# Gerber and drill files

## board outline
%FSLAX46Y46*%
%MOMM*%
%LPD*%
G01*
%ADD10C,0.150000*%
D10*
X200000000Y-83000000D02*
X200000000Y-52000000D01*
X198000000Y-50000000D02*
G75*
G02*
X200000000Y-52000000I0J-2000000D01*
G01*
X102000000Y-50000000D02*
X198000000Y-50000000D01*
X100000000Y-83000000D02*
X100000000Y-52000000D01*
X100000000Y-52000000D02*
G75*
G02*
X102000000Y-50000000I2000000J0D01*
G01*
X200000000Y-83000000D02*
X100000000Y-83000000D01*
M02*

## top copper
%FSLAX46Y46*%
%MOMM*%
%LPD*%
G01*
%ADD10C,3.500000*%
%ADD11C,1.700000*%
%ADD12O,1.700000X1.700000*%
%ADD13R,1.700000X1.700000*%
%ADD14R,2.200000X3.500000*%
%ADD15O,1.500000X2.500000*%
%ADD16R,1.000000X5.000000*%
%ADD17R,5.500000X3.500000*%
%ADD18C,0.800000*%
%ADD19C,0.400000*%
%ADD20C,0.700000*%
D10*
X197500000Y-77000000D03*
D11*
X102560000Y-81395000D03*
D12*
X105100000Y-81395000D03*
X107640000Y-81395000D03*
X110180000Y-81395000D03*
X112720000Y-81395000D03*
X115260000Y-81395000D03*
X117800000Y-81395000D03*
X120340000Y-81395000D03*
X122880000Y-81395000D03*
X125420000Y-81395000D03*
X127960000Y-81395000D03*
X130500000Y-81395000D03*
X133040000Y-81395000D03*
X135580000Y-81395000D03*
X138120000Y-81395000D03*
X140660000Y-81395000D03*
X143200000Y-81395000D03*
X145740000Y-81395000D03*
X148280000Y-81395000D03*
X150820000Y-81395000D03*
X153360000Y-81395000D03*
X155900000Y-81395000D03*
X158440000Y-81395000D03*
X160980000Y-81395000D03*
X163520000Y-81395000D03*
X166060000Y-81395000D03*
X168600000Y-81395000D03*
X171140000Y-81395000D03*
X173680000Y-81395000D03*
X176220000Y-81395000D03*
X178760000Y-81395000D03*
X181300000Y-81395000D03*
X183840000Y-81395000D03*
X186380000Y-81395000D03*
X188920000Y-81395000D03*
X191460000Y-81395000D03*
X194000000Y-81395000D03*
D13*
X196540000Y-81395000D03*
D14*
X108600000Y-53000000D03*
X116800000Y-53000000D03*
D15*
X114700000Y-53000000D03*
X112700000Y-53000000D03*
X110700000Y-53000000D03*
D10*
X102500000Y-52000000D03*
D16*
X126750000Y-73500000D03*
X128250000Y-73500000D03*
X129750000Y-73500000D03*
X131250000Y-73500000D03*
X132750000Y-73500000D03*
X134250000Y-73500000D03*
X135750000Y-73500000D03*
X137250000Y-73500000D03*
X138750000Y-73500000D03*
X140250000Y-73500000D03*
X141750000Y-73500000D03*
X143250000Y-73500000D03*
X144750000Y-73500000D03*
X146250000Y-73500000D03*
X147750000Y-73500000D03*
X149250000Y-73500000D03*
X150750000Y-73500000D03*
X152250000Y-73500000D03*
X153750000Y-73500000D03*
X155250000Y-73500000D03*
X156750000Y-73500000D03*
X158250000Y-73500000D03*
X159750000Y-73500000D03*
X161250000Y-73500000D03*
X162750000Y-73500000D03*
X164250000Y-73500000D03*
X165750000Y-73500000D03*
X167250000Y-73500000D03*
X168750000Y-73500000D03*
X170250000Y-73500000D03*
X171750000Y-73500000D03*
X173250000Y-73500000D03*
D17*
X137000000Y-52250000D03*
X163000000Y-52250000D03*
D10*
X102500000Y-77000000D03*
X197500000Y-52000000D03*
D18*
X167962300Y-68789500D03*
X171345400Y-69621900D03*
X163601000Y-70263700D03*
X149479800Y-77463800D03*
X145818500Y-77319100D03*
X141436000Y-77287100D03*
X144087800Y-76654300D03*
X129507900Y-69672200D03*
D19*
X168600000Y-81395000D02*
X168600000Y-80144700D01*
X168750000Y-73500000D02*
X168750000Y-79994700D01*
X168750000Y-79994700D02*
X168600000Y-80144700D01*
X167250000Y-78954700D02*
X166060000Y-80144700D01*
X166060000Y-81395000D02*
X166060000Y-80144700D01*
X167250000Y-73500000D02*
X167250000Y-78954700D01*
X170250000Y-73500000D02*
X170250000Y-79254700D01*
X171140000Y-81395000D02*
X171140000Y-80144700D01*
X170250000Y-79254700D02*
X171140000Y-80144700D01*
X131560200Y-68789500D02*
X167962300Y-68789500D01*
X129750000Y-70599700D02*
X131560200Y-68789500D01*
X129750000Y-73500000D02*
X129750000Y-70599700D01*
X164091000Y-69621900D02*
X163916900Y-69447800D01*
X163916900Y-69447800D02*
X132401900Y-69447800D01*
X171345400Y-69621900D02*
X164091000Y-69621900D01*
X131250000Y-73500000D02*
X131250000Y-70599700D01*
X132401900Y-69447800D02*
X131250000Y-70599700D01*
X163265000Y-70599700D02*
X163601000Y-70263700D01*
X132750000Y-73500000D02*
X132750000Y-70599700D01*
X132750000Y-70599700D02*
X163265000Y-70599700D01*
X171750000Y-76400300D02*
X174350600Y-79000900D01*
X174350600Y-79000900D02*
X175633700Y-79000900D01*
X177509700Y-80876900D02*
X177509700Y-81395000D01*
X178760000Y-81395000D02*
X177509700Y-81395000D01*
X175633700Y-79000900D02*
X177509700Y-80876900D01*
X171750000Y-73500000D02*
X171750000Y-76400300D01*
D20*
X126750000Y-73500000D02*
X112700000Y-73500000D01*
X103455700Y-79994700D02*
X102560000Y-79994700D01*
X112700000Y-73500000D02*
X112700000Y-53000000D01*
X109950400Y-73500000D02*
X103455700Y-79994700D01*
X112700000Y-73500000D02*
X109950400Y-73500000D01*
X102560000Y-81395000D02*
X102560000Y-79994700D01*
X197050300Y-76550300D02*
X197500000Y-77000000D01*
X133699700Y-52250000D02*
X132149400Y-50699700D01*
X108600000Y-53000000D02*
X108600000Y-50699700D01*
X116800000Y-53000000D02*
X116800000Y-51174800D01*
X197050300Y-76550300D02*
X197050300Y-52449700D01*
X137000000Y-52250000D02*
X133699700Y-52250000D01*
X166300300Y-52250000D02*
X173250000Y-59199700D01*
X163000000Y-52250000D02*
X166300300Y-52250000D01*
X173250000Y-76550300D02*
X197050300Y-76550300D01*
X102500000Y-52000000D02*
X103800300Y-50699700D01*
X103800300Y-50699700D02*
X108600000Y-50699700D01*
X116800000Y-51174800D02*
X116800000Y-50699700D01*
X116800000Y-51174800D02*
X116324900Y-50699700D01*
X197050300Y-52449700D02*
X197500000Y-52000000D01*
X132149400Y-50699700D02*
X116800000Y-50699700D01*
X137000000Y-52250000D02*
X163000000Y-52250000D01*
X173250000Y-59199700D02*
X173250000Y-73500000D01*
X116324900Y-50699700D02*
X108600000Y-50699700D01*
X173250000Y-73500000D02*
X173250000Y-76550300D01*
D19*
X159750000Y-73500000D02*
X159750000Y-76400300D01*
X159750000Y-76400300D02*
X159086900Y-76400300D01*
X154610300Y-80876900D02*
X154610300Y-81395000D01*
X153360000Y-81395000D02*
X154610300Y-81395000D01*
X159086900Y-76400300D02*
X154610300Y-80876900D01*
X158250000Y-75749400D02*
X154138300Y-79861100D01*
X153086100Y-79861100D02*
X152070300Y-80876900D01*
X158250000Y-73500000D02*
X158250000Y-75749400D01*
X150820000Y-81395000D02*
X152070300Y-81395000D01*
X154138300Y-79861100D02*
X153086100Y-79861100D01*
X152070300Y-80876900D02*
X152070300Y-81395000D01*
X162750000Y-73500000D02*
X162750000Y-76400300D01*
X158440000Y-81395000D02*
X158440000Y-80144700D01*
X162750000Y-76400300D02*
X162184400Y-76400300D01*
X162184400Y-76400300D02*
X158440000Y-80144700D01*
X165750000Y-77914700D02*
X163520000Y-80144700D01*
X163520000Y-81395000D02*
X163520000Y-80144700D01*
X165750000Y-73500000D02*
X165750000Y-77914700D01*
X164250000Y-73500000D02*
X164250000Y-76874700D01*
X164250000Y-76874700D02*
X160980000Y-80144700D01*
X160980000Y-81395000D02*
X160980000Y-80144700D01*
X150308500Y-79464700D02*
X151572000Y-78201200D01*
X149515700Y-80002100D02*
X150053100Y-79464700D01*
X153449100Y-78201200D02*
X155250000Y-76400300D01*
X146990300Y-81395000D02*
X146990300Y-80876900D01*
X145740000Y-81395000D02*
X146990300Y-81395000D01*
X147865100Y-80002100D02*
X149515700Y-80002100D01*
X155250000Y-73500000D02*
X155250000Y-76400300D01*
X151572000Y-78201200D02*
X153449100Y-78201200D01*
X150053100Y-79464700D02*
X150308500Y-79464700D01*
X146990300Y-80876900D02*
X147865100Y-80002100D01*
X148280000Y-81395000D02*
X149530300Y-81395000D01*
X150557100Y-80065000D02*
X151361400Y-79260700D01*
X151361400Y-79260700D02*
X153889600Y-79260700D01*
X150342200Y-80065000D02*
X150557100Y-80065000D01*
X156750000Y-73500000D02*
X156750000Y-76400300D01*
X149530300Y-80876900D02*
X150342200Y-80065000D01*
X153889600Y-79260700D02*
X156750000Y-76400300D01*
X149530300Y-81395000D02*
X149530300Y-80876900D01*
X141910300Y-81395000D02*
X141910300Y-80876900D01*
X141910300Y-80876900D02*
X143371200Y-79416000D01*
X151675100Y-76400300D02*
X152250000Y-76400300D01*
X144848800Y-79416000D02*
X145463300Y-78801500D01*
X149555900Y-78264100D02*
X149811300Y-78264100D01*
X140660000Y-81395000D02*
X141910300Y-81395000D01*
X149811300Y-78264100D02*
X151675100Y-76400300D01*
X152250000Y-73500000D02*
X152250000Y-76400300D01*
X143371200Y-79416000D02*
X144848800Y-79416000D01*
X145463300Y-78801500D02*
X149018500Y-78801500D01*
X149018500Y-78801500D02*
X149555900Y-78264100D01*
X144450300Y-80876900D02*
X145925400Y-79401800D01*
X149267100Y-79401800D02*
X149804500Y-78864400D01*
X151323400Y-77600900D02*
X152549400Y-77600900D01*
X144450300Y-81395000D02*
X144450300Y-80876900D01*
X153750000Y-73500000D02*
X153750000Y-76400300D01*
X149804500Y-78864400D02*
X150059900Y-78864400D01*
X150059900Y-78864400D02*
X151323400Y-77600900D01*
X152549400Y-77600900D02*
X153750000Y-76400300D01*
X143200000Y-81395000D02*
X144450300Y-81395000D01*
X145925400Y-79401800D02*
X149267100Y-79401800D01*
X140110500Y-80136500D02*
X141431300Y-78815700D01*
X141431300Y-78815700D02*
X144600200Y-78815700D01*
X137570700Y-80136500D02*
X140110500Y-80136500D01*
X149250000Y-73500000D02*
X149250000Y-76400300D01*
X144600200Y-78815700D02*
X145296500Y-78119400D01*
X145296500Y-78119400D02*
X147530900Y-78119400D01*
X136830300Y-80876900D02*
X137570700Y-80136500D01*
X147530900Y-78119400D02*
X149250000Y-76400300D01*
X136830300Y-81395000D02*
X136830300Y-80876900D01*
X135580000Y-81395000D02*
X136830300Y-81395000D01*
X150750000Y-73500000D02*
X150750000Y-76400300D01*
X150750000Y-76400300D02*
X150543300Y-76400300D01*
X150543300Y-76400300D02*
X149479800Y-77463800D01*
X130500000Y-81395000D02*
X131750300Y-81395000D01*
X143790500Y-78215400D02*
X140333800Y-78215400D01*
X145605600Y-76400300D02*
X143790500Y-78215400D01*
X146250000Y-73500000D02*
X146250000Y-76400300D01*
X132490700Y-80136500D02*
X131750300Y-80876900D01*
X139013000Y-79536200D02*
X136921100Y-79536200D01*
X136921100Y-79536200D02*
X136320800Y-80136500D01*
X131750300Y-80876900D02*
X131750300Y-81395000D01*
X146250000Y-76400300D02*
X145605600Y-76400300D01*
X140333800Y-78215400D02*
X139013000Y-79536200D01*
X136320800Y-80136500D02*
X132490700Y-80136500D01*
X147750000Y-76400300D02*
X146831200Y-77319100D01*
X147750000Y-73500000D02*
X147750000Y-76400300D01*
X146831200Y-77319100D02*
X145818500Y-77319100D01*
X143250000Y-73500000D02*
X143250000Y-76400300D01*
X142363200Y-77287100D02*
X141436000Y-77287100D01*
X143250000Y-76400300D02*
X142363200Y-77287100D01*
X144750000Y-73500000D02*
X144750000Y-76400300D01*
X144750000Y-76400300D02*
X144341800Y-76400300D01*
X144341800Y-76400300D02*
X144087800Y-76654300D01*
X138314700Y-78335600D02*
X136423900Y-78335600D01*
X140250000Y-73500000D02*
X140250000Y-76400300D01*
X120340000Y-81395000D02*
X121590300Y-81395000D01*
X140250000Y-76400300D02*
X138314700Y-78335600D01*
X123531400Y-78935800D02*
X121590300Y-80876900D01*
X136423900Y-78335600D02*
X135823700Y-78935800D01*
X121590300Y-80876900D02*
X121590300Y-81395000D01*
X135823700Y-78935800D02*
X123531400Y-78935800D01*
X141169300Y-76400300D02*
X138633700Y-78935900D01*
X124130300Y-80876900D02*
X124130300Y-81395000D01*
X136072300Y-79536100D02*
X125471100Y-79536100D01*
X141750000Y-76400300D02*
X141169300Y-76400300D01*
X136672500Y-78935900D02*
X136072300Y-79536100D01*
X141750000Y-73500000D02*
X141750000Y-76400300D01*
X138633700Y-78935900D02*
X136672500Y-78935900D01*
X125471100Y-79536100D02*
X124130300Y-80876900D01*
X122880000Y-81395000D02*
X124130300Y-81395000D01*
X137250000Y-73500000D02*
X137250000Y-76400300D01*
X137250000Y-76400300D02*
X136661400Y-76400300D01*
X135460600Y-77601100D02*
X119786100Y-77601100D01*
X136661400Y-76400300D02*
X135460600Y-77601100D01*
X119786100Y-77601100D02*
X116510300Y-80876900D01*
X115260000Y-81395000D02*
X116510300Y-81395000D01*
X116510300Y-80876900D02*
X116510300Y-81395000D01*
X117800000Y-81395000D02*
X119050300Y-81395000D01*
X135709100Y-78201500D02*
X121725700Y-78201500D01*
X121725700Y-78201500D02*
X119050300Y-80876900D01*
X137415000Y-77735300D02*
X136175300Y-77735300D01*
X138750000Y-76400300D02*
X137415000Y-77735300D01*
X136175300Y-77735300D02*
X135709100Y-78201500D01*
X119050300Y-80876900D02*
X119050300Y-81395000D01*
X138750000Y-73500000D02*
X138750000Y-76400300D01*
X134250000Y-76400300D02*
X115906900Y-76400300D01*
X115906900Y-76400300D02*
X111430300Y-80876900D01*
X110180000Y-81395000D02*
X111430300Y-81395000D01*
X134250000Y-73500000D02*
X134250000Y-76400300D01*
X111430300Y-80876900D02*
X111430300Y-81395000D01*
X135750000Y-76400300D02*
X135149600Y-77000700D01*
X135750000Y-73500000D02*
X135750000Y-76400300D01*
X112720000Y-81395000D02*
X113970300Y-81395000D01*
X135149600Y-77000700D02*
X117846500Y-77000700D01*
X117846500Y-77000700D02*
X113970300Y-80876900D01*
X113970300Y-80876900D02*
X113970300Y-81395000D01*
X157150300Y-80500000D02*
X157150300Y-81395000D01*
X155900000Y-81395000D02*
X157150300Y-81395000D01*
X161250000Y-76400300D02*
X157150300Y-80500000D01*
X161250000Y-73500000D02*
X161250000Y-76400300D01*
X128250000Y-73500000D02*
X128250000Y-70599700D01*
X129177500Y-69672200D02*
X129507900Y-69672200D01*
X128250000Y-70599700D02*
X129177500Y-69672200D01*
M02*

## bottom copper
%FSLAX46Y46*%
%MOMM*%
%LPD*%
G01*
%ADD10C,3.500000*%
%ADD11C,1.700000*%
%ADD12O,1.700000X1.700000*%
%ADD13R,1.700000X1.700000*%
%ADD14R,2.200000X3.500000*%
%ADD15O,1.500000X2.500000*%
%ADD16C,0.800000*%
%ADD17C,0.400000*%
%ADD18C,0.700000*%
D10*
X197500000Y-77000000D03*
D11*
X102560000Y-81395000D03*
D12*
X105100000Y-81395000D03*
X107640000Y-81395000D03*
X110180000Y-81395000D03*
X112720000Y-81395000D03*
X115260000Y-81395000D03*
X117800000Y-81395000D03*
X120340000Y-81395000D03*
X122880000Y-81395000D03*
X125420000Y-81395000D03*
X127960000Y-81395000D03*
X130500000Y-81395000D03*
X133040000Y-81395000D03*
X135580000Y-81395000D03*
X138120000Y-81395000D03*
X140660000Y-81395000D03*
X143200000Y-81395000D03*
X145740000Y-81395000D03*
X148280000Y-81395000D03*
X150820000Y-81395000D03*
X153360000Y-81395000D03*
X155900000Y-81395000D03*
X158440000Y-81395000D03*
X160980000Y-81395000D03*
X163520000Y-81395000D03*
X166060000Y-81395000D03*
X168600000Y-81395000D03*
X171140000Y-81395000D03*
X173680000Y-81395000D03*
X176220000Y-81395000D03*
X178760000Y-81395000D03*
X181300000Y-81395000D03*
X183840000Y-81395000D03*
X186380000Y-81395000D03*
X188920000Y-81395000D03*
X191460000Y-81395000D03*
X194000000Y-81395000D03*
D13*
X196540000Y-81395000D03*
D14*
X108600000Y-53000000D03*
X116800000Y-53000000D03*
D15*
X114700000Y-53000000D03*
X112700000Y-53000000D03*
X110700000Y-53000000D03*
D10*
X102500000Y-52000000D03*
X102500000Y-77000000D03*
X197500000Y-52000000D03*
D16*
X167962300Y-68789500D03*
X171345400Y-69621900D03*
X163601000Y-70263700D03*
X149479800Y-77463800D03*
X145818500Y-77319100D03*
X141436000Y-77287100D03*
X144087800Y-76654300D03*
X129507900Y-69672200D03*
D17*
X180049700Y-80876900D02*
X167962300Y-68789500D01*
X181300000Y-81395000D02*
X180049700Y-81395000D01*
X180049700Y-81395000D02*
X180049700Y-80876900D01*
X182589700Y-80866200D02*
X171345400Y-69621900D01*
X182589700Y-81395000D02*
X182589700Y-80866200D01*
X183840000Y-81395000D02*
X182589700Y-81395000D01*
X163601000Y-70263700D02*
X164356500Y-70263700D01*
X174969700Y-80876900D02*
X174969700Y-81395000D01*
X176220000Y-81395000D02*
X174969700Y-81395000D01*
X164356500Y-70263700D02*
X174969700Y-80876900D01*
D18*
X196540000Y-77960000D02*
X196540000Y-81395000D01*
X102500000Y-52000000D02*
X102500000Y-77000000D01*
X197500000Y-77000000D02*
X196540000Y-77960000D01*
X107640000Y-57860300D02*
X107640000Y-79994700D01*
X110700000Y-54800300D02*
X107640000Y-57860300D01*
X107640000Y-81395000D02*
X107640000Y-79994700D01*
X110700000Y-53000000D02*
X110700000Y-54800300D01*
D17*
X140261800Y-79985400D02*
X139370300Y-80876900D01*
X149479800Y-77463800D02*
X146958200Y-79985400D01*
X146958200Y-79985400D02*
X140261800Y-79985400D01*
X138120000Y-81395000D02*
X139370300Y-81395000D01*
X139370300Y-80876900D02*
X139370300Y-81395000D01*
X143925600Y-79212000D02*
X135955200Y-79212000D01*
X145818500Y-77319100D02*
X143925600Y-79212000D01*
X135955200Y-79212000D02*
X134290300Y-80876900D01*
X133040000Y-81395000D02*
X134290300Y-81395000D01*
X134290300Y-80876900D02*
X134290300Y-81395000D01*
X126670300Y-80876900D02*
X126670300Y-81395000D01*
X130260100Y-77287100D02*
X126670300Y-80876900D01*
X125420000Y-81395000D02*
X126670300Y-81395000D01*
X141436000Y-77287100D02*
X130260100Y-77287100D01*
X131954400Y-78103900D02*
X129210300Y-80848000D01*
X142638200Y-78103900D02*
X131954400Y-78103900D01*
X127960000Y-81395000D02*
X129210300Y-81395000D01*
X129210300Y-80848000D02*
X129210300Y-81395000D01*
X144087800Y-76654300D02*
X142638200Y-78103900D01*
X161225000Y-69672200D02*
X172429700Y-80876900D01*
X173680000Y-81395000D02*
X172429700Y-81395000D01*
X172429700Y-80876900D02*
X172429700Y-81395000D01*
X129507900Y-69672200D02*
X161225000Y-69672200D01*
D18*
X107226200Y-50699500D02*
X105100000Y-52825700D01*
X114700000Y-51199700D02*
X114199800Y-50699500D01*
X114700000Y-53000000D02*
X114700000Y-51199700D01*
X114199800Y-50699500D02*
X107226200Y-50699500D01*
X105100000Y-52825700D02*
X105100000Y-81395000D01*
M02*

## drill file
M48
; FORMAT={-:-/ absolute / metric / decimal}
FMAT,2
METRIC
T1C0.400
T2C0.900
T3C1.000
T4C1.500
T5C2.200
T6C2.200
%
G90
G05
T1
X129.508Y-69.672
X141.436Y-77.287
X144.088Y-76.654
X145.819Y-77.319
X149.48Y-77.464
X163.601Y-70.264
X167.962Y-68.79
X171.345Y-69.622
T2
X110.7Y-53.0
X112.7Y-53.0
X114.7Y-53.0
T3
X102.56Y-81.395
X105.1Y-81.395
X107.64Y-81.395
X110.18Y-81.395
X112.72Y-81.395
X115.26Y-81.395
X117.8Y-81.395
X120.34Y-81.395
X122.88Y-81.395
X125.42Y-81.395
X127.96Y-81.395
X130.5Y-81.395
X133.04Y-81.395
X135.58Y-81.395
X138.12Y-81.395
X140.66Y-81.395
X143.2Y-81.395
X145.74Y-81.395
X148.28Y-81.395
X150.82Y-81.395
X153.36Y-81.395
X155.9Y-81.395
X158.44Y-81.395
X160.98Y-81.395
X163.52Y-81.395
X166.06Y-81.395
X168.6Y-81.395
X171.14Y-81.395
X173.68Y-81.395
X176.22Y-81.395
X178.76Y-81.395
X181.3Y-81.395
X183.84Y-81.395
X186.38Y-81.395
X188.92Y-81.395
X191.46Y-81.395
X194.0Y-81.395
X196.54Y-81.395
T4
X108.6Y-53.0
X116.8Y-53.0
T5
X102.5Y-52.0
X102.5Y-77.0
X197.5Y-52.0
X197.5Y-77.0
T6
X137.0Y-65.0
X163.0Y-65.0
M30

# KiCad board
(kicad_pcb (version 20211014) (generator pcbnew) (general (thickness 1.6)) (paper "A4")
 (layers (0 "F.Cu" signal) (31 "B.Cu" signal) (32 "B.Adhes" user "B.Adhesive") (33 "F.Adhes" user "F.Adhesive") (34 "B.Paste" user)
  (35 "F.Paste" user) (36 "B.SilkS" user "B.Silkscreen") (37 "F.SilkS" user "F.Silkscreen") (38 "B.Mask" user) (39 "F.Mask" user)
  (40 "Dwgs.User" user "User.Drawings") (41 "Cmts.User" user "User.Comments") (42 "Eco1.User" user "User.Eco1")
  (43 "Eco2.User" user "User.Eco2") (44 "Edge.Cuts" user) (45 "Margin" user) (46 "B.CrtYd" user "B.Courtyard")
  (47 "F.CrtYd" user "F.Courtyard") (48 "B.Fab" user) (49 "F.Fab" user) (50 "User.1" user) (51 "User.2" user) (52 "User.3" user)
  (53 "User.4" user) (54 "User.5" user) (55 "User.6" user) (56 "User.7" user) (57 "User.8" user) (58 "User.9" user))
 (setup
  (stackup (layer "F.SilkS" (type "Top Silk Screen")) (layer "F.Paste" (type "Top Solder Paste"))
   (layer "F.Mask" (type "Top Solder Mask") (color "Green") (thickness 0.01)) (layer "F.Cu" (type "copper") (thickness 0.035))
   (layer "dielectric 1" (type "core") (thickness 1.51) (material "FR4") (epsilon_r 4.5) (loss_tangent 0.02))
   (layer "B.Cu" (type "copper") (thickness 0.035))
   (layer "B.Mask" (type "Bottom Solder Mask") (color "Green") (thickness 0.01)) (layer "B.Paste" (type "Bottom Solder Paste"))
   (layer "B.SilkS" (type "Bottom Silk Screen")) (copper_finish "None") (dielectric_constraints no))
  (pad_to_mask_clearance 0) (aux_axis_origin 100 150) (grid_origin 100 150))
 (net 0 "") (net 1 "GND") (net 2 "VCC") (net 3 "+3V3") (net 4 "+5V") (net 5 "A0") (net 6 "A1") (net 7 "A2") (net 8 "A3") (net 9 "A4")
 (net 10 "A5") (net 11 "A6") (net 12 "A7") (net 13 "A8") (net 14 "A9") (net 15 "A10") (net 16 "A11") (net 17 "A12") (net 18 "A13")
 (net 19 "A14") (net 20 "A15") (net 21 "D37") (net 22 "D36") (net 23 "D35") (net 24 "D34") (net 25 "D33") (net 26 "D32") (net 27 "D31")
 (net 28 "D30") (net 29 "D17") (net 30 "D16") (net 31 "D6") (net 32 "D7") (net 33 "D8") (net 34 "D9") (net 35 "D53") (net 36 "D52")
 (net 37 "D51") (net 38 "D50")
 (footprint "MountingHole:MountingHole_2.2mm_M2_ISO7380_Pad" (layer "F.Cu") (at 197.5 77)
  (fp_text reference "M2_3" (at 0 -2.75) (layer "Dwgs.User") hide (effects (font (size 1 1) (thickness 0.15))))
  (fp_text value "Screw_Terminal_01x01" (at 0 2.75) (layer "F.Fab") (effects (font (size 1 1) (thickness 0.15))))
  (pad "1" thru_hole circle locked (at 0 0) (size 3.5 3.5) (drill 2.2) (layers *.Cu *.Mask) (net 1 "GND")))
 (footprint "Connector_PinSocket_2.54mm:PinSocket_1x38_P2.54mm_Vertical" (layer "F.Cu") (at 102.56 81.395 90)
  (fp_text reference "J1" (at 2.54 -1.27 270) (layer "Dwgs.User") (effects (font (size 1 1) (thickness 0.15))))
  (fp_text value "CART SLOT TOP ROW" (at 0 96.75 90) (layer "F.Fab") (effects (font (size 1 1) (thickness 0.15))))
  (pad "1" thru_hole circle (at 0 0 90) (size 1.7 1.7) (drill 1) (layers *.Cu *.Mask) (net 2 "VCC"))
  (pad "2" thru_hole oval (at 0 2.54 90) (size 1.7 1.7) (drill 1) (layers *.Cu *.Mask) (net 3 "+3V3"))
  (pad "3" thru_hole oval (at 0 5.08 90) (size 1.7 1.7) (drill 1) (layers *.Cu *.Mask) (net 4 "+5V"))
  (pad "4" thru_hole oval (at 0 7.62 90) (size 1.7 1.7) (drill 1) (layers *.Cu *.Mask) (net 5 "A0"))
  (pad "5" thru_hole oval (at 0 10.16 90) (size 1.7 1.7) (drill 1) (layers *.Cu *.Mask) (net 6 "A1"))
  (pad "6" thru_hole oval (at 0 12.7 90) (size 1.7 1.7) (drill 1) (layers *.Cu *.Mask) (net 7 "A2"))
  (pad "7" thru_hole oval (at 0 15.24 90) (size 1.7 1.7) (drill 1) (layers *.Cu *.Mask) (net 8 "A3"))
  (pad "8" thru_hole oval (at 0 17.78 90) (size 1.7 1.7) (drill 1) (layers *.Cu *.Mask) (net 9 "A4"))
  (pad "9" thru_hole oval (at 0 20.32 90) (size 1.7 1.7) (drill 1) (layers *.Cu *.Mask) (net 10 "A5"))
  (pad "10" thru_hole oval (at 0 22.86 90) (size 1.7 1.7) (drill 1) (layers *.Cu *.Mask) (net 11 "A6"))
  (pad "11" thru_hole oval (at 0 25.4 90) (size 1.7 1.7) (drill 1) (layers *.Cu *.Mask) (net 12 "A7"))
  (pad "12" thru_hole oval (at 0 27.94 90) (size 1.7 1.7) (drill 1) (layers *.Cu *.Mask) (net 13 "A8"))
  (pad "13" thru_hole oval (at 0 30.48 90) (size 1.7 1.7) (drill 1) (layers *.Cu *.Mask) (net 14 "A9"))
  (pad "14" thru_hole oval (at 0 33.02 90) (size 1.7 1.7) (drill 1) (layers *.Cu *.Mask) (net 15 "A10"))
  (pad "15" thru_hole oval (at 0 35.56 90) (size 1.7 1.7) (drill 1) (layers *.Cu *.Mask) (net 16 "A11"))
  (pad "16" thru_hole oval (at 0 38.1 90) (size 1.7 1.7) (drill 1) (layers *.Cu *.Mask) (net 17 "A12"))
  (pad "17" thru_hole oval (at 0 40.64 90) (size 1.7 1.7) (drill 1) (layers *.Cu *.Mask) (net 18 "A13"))
  (pad "18" thru_hole oval (at 0 43.18 90) (size 1.7 1.7) (drill 1) (layers *.Cu *.Mask) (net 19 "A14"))
  (pad "19" thru_hole oval (at 0 45.72 90) (size 1.7 1.7) (drill 1) (layers *.Cu *.Mask) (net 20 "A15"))
  (pad "20" thru_hole oval (at 0 48.26 90) (size 1.7 1.7) (drill 1) (layers *.Cu *.Mask) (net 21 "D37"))
  (pad "21" thru_hole oval (at 0 50.8 90) (size 1.7 1.7) (drill 1) (layers *.Cu *.Mask) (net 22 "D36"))
  (pad "22" thru_hole oval (at 0 53.34 90) (size 1.7 1.7) (drill 1) (layers *.Cu *.Mask) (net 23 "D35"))
  (pad "23" thru_hole oval (at 0 55.88 90) (size 1.7 1.7) (drill 1) (layers *.Cu *.Mask) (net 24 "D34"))
  (pad "24" thru_hole oval (at 0 58.42 90) (size 1.7 1.7) (drill 1) (layers *.Cu *.Mask) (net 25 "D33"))
  (pad "25" thru_hole oval (at 0 60.96 90) (size 1.7 1.7) (drill 1) (layers *.Cu *.Mask) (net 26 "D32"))
  (pad "26" thru_hole oval (at 0 63.5 90) (size 1.7 1.7) (drill 1) (layers *.Cu *.Mask) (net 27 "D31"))
  (pad "27" thru_hole oval (at 0 66.04 90) (size 1.7 1.7) (drill 1) (layers *.Cu *.Mask) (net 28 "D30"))
  (pad "28" thru_hole oval (at 0 68.58 90) (size 1.7 1.7) (drill 1) (layers *.Cu *.Mask) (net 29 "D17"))
  (pad "29" thru_hole oval (at 0 71.12 90) (size 1.7 1.7) (drill 1) (layers *.Cu *.Mask) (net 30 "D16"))
  (pad "30" thru_hole oval (at 0 73.66 90) (size 1.7 1.7) (drill 1) (layers *.Cu *.Mask) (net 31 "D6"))
  (pad "31" thru_hole oval (at 0 76.2 90) (size 1.7 1.7) (drill 1) (layers *.Cu *.Mask) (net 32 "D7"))
  (pad "32" thru_hole oval (at 0 78.74 90) (size 1.7 1.7) (drill 1) (layers *.Cu *.Mask) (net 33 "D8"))
  (pad "33" thru_hole oval (at 0 81.28 90) (size 1.7 1.7) (drill 1) (layers *.Cu *.Mask) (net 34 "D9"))
  (pad "34" thru_hole oval (at 0 83.82 90) (size 1.7 1.7) (drill 1) (layers *.Cu *.Mask) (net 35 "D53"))
  (pad "35" thru_hole oval (at 0 86.36 90) (size 1.7 1.7) (drill 1) (layers *.Cu *.Mask) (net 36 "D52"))
  (pad "36" thru_hole oval (at 0 88.9 90) (size 1.7 1.7) (drill 1) (layers *.Cu *.Mask) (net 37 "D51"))
  (pad "37" thru_hole oval (at 0 91.44 90) (size 1.7 1.7) (drill 1) (layers *.Cu *.Mask) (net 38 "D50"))
  (pad "38" thru_hole rect (at 0 93.98 90) (size 1.7 1.7) (drill 1) (layers *.Cu *.Mask) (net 1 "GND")))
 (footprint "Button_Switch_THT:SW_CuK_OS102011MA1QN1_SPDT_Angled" (layer "F.Cu") (at 114.7 53 180)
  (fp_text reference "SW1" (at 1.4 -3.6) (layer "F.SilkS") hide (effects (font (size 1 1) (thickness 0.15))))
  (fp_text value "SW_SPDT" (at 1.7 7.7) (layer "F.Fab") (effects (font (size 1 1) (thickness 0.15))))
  (pad "" thru_hole rect (at 6.1 0 180) (size 2.2 3.5) (drill 1.5) (layers *.Cu *.Mask) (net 1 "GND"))
  (pad "" thru_hole rect (at -2.1 0 180) (size 2.2 3.5) (drill 1.5) (layers *.Cu *.Mask) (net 1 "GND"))
  (pad "1" thru_hole oval (at 0 0 180) (size 1.5 2.5) (drill 0.9) (layers *.Cu *.Mask) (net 3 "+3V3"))
  (pad "2" thru_hole oval (at 2 0 180) (size 1.5 2.5) (drill 0.9) (layers *.Cu *.Mask) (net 2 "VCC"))
  (pad "3" thru_hole oval (at 4 0 180) (size 1.5 2.5) (drill 0.9) (layers *.Cu *.Mask) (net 4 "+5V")))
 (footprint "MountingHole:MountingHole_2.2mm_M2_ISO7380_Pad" (layer "F.Cu") (at 102.5 52)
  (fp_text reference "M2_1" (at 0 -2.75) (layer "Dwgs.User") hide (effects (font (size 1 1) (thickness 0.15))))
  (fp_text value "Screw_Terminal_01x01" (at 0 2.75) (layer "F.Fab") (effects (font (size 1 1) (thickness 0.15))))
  (pad "1" thru_hole circle locked (at 0 0) (size 3.5 3.5) (drill 2.2) (layers *.Cu *.Mask) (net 1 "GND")))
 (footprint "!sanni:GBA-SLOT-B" (layer "F.Cu") (at 150 68.5 90)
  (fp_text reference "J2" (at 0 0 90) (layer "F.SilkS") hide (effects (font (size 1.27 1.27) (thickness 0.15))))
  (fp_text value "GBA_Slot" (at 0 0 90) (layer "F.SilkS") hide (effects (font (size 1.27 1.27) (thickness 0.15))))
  (pad "" np_thru_hole circle locked (at 3.5 -13 90) (size 2.2 2.2) (drill 2.2) (layers *.Cu *.Mask))
  (pad "" np_thru_hole circle locked (at 3.5 13 90) (size 2.2 2.2) (drill 2.2) (layers *.Cu *.Mask))
  (pad "1" smd rect locked (at -5 -23.25 270) (size 5 1) (layers "F.Cu" "F.Paste" "F.Mask") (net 2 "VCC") (solder_mask_margin 0.0508))
  (pad "2" smd rect locked (at -5 -21.75 270) (size 5 1) (layers "F.Cu" "F.Paste" "F.Mask") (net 30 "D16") (solder_mask_margin 0.0508))
  (pad "3" smd rect locked (at -5 -20.25 270) (size 5 1) (layers "F.Cu" "F.Paste" "F.Mask") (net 33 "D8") (solder_mask_margin 0.0508))
  (pad "4" smd rect locked (at -5 -18.75 270) (size 5 1) (layers "F.Cu" "F.Paste" "F.Mask") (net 34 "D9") (solder_mask_margin 0.0508))
  (pad "5" smd rect locked (at -5 -17.25 270) (size 5 1) (layers "F.Cu" "F.Paste" "F.Mask") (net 31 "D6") (solder_mask_margin 0.0508))
  (pad "6" smd rect locked (at -5 -15.75 270) (size 5 1) (layers "F.Cu" "F.Paste" "F.Mask") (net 5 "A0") (solder_mask_margin 0.0508))
  (pad "7" smd rect locked (at -5 -14.25 270) (size 5 1) (layers "F.Cu" "F.Paste" "F.Mask") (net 6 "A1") (solder_mask_margin 0.0508))
  (pad "8" smd rect locked (at -5 -12.75 270) (size 5 1) (layers "F.Cu" "F.Paste" "F.Mask") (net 7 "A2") (solder_mask_margin 0.0508))
  (pad "9" smd rect locked (at -5 -11.25 270) (size 5 1) (layers "F.Cu" "F.Paste" "F.Mask") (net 8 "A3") (solder_mask_margin 0.0508))
  (pad "10" smd rect locked (at -5 -9.75 270) (size 5 1) (layers "F.Cu" "F.Paste" "F.Mask") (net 9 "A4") (solder_mask_margin 0.0508))
  (pad "11" smd rect locked (at -5 -8.25 270) (size 5 1) (layers "F.Cu" "F.Paste" "F.Mask") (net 10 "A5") (solder_mask_margin 0.0508))
  (pad "12" smd rect locked (at -5 -6.75 270) (size 5 1) (layers "F.Cu" "F.Paste" "F.Mask") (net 11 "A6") (solder_mask_margin 0.0508))
  (pad "13" smd rect locked (at -5 -5.25 270) (size 5 1) (layers "F.Cu" "F.Paste" "F.Mask") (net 12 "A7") (solder_mask_margin 0.0508))
  (pad "14" smd rect locked (at -5 -3.75 270) (size 5 1) (layers "F.Cu" "F.Paste" "F.Mask") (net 13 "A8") (solder_mask_margin 0.0508))
  (pad "15" smd rect locked (at -5 -2.25 270) (size 5 1) (layers "F.Cu" "F.Paste" "F.Mask") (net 14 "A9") (solder_mask_margin 0.0508))
  (pad "16" smd rect locked (at -5 -0.75 270) (size 5 1) (layers "F.Cu" "F.Paste" "F.Mask") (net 15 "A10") (solder_mask_margin 0.0508))
  (pad "17" smd rect locked (at -5 0.75 270) (size 5 1) (layers "F.Cu" "F.Paste" "F.Mask") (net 16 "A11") (solder_mask_margin 0.0508))
  (pad "18" smd rect locked (at -5 2.25 270) (size 5 1) (layers "F.Cu" "F.Paste" "F.Mask") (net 17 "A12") (solder_mask_margin 0.0508))
  (pad "19" smd rect locked (at -5 3.75 270) (size 5 1) (layers "F.Cu" "F.Paste" "F.Mask") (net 18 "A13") (solder_mask_margin 0.0508))
  (pad "20" smd rect locked (at -5 5.25 270) (size 5 1) (layers "F.Cu" "F.Paste" "F.Mask") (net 19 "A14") (solder_mask_margin 0.0508))
  (pad "21" smd rect locked (at -5 6.75 270) (size 5 1) (layers "F.Cu" "F.Paste" "F.Mask") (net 20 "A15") (solder_mask_margin 0.0508))
  (pad "22" smd rect locked (at -5 8.25 270) (size 5 1) (layers "F.Cu" "F.Paste" "F.Mask") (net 21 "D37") (solder_mask_margin 0.0508))
  (pad "23" smd rect locked (at -5 9.75 270) (size 5 1) (layers "F.Cu" "F.Paste" "F.Mask") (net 22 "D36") (solder_mask_margin 0.0508))
  (pad "24" smd rect locked (at -5 11.25 270) (size 5 1) (layers "F.Cu" "F.Paste" "F.Mask") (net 23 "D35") (solder_mask_margin 0.0508))
  (pad "25" smd rect locked (at -5 12.75 270) (size 5 1) (layers "F.Cu" "F.Paste" "F.Mask") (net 24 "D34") (solder_mask_margin 0.0508))
  (pad "26" smd rect locked (at -5 14.25 270) (size 5 1) (layers "F.Cu" "F.Paste" "F.Mask") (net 25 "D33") (solder_mask_margin 0.0508))
  (pad "27" smd rect locked (at -5 15.75 270) (size 5 1) (layers "F.Cu" "F.Paste" "F.Mask") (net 26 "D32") (solder_mask_margin 0.0508))
  (pad "28" smd rect locked (at -5 17.25 270) (size 5 1) (layers "F.Cu" "F.Paste" "F.Mask") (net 27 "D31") (solder_mask_margin 0.0508))
  (pad "29" smd rect locked (at -5 18.75 270) (size 5 1) (layers "F.Cu" "F.Paste" "F.Mask") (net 28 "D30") (solder_mask_margin 0.0508))
  (pad "30" smd rect locked (at -5 20.25 270) (size 5 1) (layers "F.Cu" "F.Paste" "F.Mask") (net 29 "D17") (solder_mask_margin 0.0508))
  (pad "31" smd rect locked (at -5 21.75 270) (size 5 1) (layers "F.Cu" "F.Paste" "F.Mask") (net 32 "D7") (solder_mask_margin 0.0508))
  (pad "32" smd rect locked (at -5 23.25 270) (size 5 1) (layers "F.Cu" "F.Paste" "F.Mask") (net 1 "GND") (solder_mask_margin 0.0508))
  (pad "SHIELD_3" smd rect locked (at 16.25 -13) (size 5.5 3.5) (layers "F.Cu" "F.Paste" "F.Mask") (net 1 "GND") (solder_mask_margin 0.0508))
  (pad "SHIELD_4" smd rect locked (at 16.25 13) (size 5.5 3.5) (layers "F.Cu" "F.Paste" "F.Mask") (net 1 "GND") (solder_mask_margin 0.0508)))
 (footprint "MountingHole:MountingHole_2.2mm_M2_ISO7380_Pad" (layer "F.Cu") (at 102.5 77)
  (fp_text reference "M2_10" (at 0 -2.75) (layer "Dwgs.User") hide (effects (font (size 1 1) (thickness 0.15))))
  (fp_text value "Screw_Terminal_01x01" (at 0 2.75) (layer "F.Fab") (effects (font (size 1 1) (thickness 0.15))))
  (pad "1" thru_hole circle locked (at 0 0) (size 3.5 3.5) (drill 2.2) (layers *.Cu *.Mask) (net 1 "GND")))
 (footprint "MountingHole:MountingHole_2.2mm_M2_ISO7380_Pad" (layer "F.Cu") (at 197.5 52)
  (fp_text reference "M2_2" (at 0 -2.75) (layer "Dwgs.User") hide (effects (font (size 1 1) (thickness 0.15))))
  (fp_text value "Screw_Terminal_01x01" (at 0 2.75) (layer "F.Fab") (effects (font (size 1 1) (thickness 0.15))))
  (pad "1" thru_hole circle locked (at 0 0) (size 3.5 3.5) (drill 2.2) (layers *.Cu *.Mask) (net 1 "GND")))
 (gr_line (start 200 83) (end 200 52) (layer "Edge.Cuts") (width 0.15))
 (gr_arc (start 198 50) (mid 199.414214 50.585786) (end 200.000001 52) (layer "Edge.Cuts") (width 0.15))
 (gr_line (start 102 50) (end 198 50) (layer "Edge.Cuts") (width 0.15))
 (gr_line (start 100 83) (end 100 52) (layer "Edge.Cuts") (width 0.15))
 (gr_arc (start 100 52) (mid 100.585786 50.585786) (end 102 50) (layer "Edge.Cuts") (width 0.15))
 (gr_line (start 200 83) (end 100 83) (layer "Edge.Cuts") (width 0.15))
 (segment (start 168.6 81.395) (end 168.6 80.1447) (width 0.4) (layer "F.Cu") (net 28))
 (segment (start 168.75 73.5) (end 168.75 79.9947) (width 0.4) (layer "F.Cu") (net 28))
 (segment (start 168.75 79.9947) (end 168.6 80.1447) (width 0.4) (layer "F.Cu") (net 28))
 (segment (start 167.25 78.9547) (end 166.06 80.1447) (width 0.4) (layer "F.Cu") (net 27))
 (segment (start 166.06 81.395) (end 166.06 80.1447) (width 0.4) (layer "F.Cu") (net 27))
 (segment (start 167.25 73.5) (end 167.25 78.9547) (width 0.4) (layer "F.Cu") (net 27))
 (segment (start 170.25 73.5) (end 170.25 79.2547) (width 0.4) (layer "F.Cu") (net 29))
 (segment (start 171.14 81.395) (end 171.14 80.1447) (width 0.4) (layer "F.Cu") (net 29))
 (segment (start 170.25 79.2547) (end 171.14 80.1447) (width 0.4) (layer "F.Cu") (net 29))
 (segment (start 131.5602 68.7895) (end 167.9623 68.7895) (width 0.4) (layer "F.Cu") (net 33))
 (segment (start 129.75 70.5997) (end 131.5602 68.7895) (width 0.4) (layer "F.Cu") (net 33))
 (segment (start 129.75 73.5) (end 129.75 70.5997) (width 0.4) (layer "F.Cu") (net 33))
 (via (at 167.9623 68.7895) (size 0.8) (drill 0.4) (layers "F.Cu" "B.Cu") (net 33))
 (segment (start 180.0497 80.8769) (end 167.9623 68.7895) (width 0.4) (layer "B.Cu") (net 33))
 (segment (start 181.3 81.395) (end 180.0497 81.395) (width 0.4) (layer "B.Cu") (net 33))
 (segment (start 180.0497 81.395) (end 180.0497 80.8769) (width 0.4) (layer "B.Cu") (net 33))
 (segment (start 164.091 69.6219) (end 163.9169 69.4478) (width 0.4) (layer "F.Cu") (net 34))
 (segment (start 163.9169 69.4478) (end 132.4019 69.4478) (width 0.4) (layer "F.Cu") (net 34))
 (segment (start 171.3454 69.6219) (end 164.091 69.6219) (width 0.4) (layer "F.Cu") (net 34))
 (segment (start 131.25 73.5) (end 131.25 70.5997) (width 0.4) (layer "F.Cu") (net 34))
 (segment (start 132.4019 69.4478) (end 131.25 70.5997) (width 0.4) (layer "F.Cu") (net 34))
 (via (at 171.3454 69.6219) (size 0.8) (drill 0.4) (layers "F.Cu" "B.Cu") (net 34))
 (segment (start 182.5897 80.8662) (end 171.3454 69.6219) (width 0.4) (layer "B.Cu") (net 34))
 (segment (start 182.5897 81.395) (end 182.5897 80.8662) (width 0.4) (layer "B.Cu") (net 34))
 (segment (start 183.84 81.395) (end 182.5897 81.395) (width 0.4) (layer "B.Cu") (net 34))
 (segment (start 163.265 70.5997) (end 163.601 70.2637) (width 0.4) (layer "F.Cu") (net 31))
 (segment (start 132.75 73.5) (end 132.75 70.5997) (width 0.4) (layer "F.Cu") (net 31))
 (segment (start 132.75 70.5997) (end 163.265 70.5997) (width 0.4) (layer "F.Cu") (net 31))
 (via (at 163.601 70.2637) (size 0.8) (drill 0.4) (layers "F.Cu" "B.Cu") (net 31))
 (segment (start 163.601 70.2637) (end 164.3565 70.2637) (width 0.4) (layer "B.Cu") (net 31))
 (segment (start 174.9697 80.8769) (end 174.9697 81.395) (width 0.4) (layer "B.Cu") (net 31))
 (segment (start 176.22 81.395) (end 174.9697 81.395) (width 0.4) (layer "B.Cu") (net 31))
 (segment (start 164.3565 70.2637) (end 174.9697 80.8769) (width 0.4) (layer "B.Cu") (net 31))
 (segment (start 171.75 76.4003) (end 174.3506 79.0009) (width 0.4) (layer "F.Cu") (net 32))
 (segment (start 174.3506 79.0009) (end 175.6337 79.0009) (width 0.4) (layer "F.Cu") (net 32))
 (segment (start 177.5097 80.8769) (end 177.5097 81.395) (width 0.4) (layer "F.Cu") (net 32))
 (segment (start 178.76 81.395) (end 177.5097 81.395) (width 0.4) (layer "F.Cu") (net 32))
 (segment (start 175.6337 79.0009) (end 177.5097 80.8769) (width 0.4) (layer "F.Cu") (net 32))
 (segment (start 171.75 73.5) (end 171.75 76.4003) (width 0.4) (layer "F.Cu") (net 32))
 (segment (start 126.75 73.5) (end 112.7 73.5) (width 0.7) (layer "F.Cu") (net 2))
 (segment (start 103.4557 79.9947) (end 102.56 79.9947) (width 0.7) (layer "F.Cu") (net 2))
 (segment (start 112.7 73.5) (end 112.7 53) (width 0.7) (layer "F.Cu") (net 2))
 (segment (start 109.9504 73.5) (end 103.4557 79.9947) (width 0.7) (layer "F.Cu") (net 2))
 (segment (start 112.7 73.5) (end 109.9504 73.5) (width 0.7) (layer "F.Cu") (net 2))
 (segment (start 102.56 81.395) (end 102.56 79.9947) (width 0.7) (layer "F.Cu") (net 2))
 (segment (start 197.0503 76.5503) (end 197.5 77) (width 0.7) (layer "F.Cu") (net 1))
 (segment (start 133.6997 52.25) (end 132.1494 50.6997) (width 0.7) (layer "F.Cu") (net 1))
 (segment (start 108.6 53) (end 108.6 50.6997) (width 0.7) (layer "F.Cu") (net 1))
 (segment (start 116.8 53) (end 116.8 51.1748) (width 0.7) (layer "F.Cu") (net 1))
 (segment (start 197.0503 76.5503) (end 197.0503 52.4497) (width 0.7) (layer "F.Cu") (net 1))
 (segment (start 137 52.25) (end 133.6997 52.25) (width 0.7) (layer "F.Cu") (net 1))
 (segment (start 166.3003 52.25) (end 173.25 59.1997) (width 0.7) (layer "F.Cu") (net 1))
 (segment (start 163 52.25) (end 166.3003 52.25) (width 0.7) (layer "F.Cu") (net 1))
 (segment (start 173.25 76.5503) (end 197.0503 76.5503) (width 0.7) (layer "F.Cu") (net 1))
 (segment (start 102.5 52) (end 103.8003 50.6997) (width 0.7) (layer "F.Cu") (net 1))
 (segment (start 103.8003 50.6997) (end 108.6 50.6997) (width 0.7) (layer "F.Cu") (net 1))
 (segment (start 116.8 51.1748) (end 116.8 50.6997) (width 0.7) (layer "F.Cu") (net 1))
 (segment (start 116.8 51.1748) (end 116.3249 50.6997) (width 0.7) (layer "F.Cu") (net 1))
 (segment (start 197.0503 52.4497) (end 197.5 52) (width 0.7) (layer "F.Cu") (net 1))
 (segment (start 132.1494 50.6997) (end 116.8 50.6997) (width 0.7) (layer "F.Cu") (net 1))
 (segment (start 137 52.25) (end 163 52.25) (width 0.7) (layer "F.Cu") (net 1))
 (segment (start 173.25 59.1997) (end 173.25 73.5) (width 0.7) (layer "F.Cu") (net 1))
 (segment (start 116.3249 50.6997) (end 108.6 50.6997) (width 0.7) (layer "F.Cu") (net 1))
 (segment (start 173.25 73.5) (end 173.25 76.5503) (width 0.7) (layer "F.Cu") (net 1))
 (segment (start 196.54 77.96) (end 196.54 81.395) (width 0.7) (layer "B.Cu") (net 1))
 (segment (start 102.5 52) (end 102.5 77) (width 0.7) (layer "B.Cu") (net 1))
 (segment (start 197.5 77) (end 196.54 77.96) (width 0.7) (layer "B.Cu") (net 1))
 (segment (start 107.64 57.8603) (end 107.64 79.9947) (width 0.7) (layer "B.Cu") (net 4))
 (segment (start 110.7 54.8003) (end 107.64 57.8603) (width 0.7) (layer "B.Cu") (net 4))
 (segment (start 107.64 81.395) (end 107.64 79.9947) (width 0.7) (layer "B.Cu") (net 4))
 (segment (start 110.7 53) (end 110.7 54.8003) (width 0.7) (layer "B.Cu") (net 4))
 (segment (start 159.75 73.5) (end 159.75 76.4003) (width 0.4) (layer "F.Cu") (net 22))
 (segment (start 159.75 76.4003) (end 159.0869 76.4003) (width 0.4) (layer "F.Cu") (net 22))
 (segment (start 154.6103 80.8769) (end 154.6103 81.395) (width 0.4) (layer "F.Cu") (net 22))
 (segment (start 153.36 81.395) (end 154.6103 81.395) (width 0.4) (layer "F.Cu") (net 22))
 (segment (start 159.0869 76.4003) (end 154.6103 80.8769) (width 0.4) (layer "F.Cu") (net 22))
 (segment (start 158.25 75.7494) (end 154.1383 79.8611) (width 0.4) (layer "F.Cu") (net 21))
 (segment (start 153.0861 79.8611) (end 152.0703 80.8769) (width 0.4) (layer "F.Cu") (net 21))
 (segment (start 158.25 73.5) (end 158.25 75.7494) (width 0.4) (layer "F.Cu") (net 21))
 (segment (start 150.82 81.395) (end 152.0703 81.395) (width 0.4) (layer "F.Cu") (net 21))
 (segment (start 154.1383 79.8611) (end 153.0861 79.8611) (width 0.4) (layer "F.Cu") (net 21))
 (segment (start 152.0703 80.8769) (end 152.0703 81.395) (width 0.4) (layer "F.Cu") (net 21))
 (segment (start 162.75 73.5) (end 162.75 76.4003) (width 0.4) (layer "F.Cu") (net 24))
 (segment (start 158.44 81.395) (end 158.44 80.1447) (width 0.4) (layer "F.Cu") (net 24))
 (segment (start 162.75 76.4003) (end 162.1844 76.4003) (width 0.4) (layer "F.Cu") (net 24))
 (segment (start 162.1844 76.4003) (end 158.44 80.1447) (width 0.4) (layer "F.Cu") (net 24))
 (segment (start 165.75 77.9147) (end 163.52 80.1447) (width 0.4) (layer "F.Cu") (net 26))
 (segment (start 163.52 81.395) (end 163.52 80.1447) (width 0.4) (layer "F.Cu") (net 26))
 (segment (start 165.75 73.5) (end 165.75 77.9147) (width 0.4) (layer "F.Cu") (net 26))
 (segment (start 164.25 73.5) (end 164.25 76.8747) (width 0.4) (layer "F.Cu") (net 25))
 (segment (start 164.25 76.8747) (end 160.98 80.1447) (width 0.4) (layer "F.Cu") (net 25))
 (segment (start 160.98 81.395) (end 160.98 80.1447) (width 0.4) (layer "F.Cu") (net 25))
 (segment (start 150.3085 79.4647) (end 151.572 78.2012) (width 0.4) (layer "F.Cu") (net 19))
 (segment (start 149.5157 80.0021) (end 150.0531 79.4647) (width 0.4) (layer "F.Cu") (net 19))
 (segment (start 153.4491 78.2012) (end 155.25 76.4003) (width 0.4) (layer "F.Cu") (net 19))
 (segment (start 146.9903 81.395) (end 146.9903 80.8769) (width 0.4) (layer "F.Cu") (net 19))
 (segment (start 145.74 81.395) (end 146.9903 81.395) (width 0.4) (layer "F.Cu") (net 19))
 (segment (start 147.8651 80.0021) (end 149.5157 80.0021) (width 0.4) (layer "F.Cu") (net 19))
 (segment (start 155.25 73.5) (end 155.25 76.4003) (width 0.4) (layer "F.Cu") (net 19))
 (segment (start 151.572 78.2012) (end 153.4491 78.2012) (width 0.4) (layer "F.Cu") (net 19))
 (segment (start 150.0531 79.4647) (end 150.3085 79.4647) (width 0.4) (layer "F.Cu") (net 19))
 (segment (start 146.9903 80.8769) (end 147.8651 80.0021) (width 0.4) (layer "F.Cu") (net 19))
 (segment (start 148.28 81.395) (end 149.5303 81.395) (width 0.4) (layer "F.Cu") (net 20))
 (segment (start 150.5571 80.065) (end 151.3614 79.2607) (width 0.4) (layer "F.Cu") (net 20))
 (segment (start 151.3614 79.2607) (end 153.8896 79.2607) (width 0.4) (layer "F.Cu") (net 20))
 (segment (start 150.3422 80.065) (end 150.5571 80.065) (width 0.4) (layer "F.Cu") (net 20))
 (segment (start 156.75 73.5) (end 156.75 76.4003) (width 0.4) (layer "F.Cu") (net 20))
 (segment (start 149.5303 80.8769) (end 150.3422 80.065) (width 0.4) (layer "F.Cu") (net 20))
 (segment (start 153.8896 79.2607) (end 156.75 76.4003) (width 0.4) (layer "F.Cu") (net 20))
 (segment (start 149.5303 81.395) (end 149.5303 80.8769) (width 0.4) (layer "F.Cu") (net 20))
 (segment (start 141.9103 81.395) (end 141.9103 80.8769) (width 0.4) (layer "F.Cu") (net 17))
 (segment (start 141.9103 80.8769) (end 143.3712 79.416) (width 0.4) (layer "F.Cu") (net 17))
 (segment (start 151.6751 76.4003) (end 152.25 76.4003) (width 0.4) (layer "F.Cu") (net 17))
 (segment (start 144.8488 79.416) (end 145.4633 78.8015) (width 0.4) (layer "F.Cu") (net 17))
 (segment (start 149.5559 78.2641) (end 149.8113 78.2641) (width 0.4) (layer "F.Cu") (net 17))
 (segment (start 140.66 81.395) (end 141.9103 81.395) (width 0.4) (layer "F.Cu") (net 17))
 (segment (start 149.8113 78.2641) (end 151.6751 76.4003) (width 0.4) (layer "F.Cu") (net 17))
 (segment (start 152.25 73.5) (end 152.25 76.4003) (width 0.4) (layer "F.Cu") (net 17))
 (segment (start 143.3712 79.416) (end 144.8488 79.416) (width 0.4) (layer "F.Cu") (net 17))
 (segment (start 145.4633 78.8015) (end 149.0185 78.8015) (width 0.4) (layer "F.Cu") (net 17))
 (segment (start 149.0185 78.8015) (end 149.5559 78.2641) (width 0.4) (layer "F.Cu") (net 17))
 (segment (start 144.4503 80.8769) (end 145.9254 79.4018) (width 0.4) (layer "F.Cu") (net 18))
 (segment (start 149.2671 79.4018) (end 149.8045 78.8644) (width 0.4) (layer "F.Cu") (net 18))
 (segment (start 151.3234 77.6009) (end 152.5494 77.6009) (width 0.4) (layer "F.Cu") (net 18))
 (segment (start 144.4503 81.395) (end 144.4503 80.8769) (width 0.4) (layer "F.Cu") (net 18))
 (segment (start 153.75 73.5) (end 153.75 76.4003) (width 0.4) (layer "F.Cu") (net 18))
 (segment (start 149.8045 78.8644) (end 150.0599 78.8644) (width 0.4) (layer "F.Cu") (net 18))
 (segment (start 150.0599 78.8644) (end 151.3234 77.6009) (width 0.4) (layer "F.Cu") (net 18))
 (segment (start 152.5494 77.6009) (end 153.75 76.4003) (width 0.4) (layer "F.Cu") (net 18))
 (segment (start 143.2 81.395) (end 144.4503 81.395) (width 0.4) (layer "F.Cu") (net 18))
 (segment (start 145.9254 79.4018) (end 149.2671 79.4018) (width 0.4) (layer "F.Cu") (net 18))
 (segment (start 140.1105 80.1365) (end 141.4313 78.8157) (width 0.4) (layer "F.Cu") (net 15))
 (segment (start 141.4313 78.8157) (end 144.6002 78.8157) (width 0.4) (layer "F.Cu") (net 15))
 (segment (start 137.5707 80.1365) (end 140.1105 80.1365) (width 0.4) (layer "F.Cu") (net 15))
 (segment (start 149.25 73.5) (end 149.25 76.4003) (width 0.4) (layer "F.Cu") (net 15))
 (segment (start 144.6002 78.8157) (end 145.2965 78.1194) (width 0.4) (layer "F.Cu") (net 15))
 (segment (start 145.2965 78.1194) (end 147.5309 78.1194) (width 0.4) (layer "F.Cu") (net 15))
 (segment (start 136.8303 80.8769) (end 137.5707 80.1365) (width 0.4) (layer "F.Cu") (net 15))
 (segment (start 147.5309 78.1194) (end 149.25 76.4003) (width 0.4) (layer "F.Cu") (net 15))
 (segment (start 136.8303 81.395) (end 136.8303 80.8769) (width 0.4) (layer "F.Cu") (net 15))
 (segment (start 135.58 81.395) (end 136.8303 81.395) (width 0.4) (layer "F.Cu") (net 15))
 (segment (start 150.75 73.5) (end 150.75 76.4003) (width 0.4) (layer "F.Cu") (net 16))
 (segment (start 150.75 76.4003) (end 150.5433 76.4003) (width 0.4) (layer "F.Cu") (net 16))
 (segment (start 150.5433 76.4003) (end 149.4798 77.4638) (width 0.4) (layer "F.Cu") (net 16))
 (via (at 149.4798 77.4638) (size 0.8) (drill 0.4) (layers "F.Cu" "B.Cu") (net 16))
 (segment (start 140.2618 79.9854) (end 139.3703 80.8769) (width 0.4) (layer "B.Cu") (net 16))
 (segment (start 149.4798 77.4638) (end 146.9582 79.9854) (width 0.4) (layer "B.Cu") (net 16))
 (segment (start 146.9582 79.9854) (end 140.2618 79.9854) (width 0.4) (layer "B.Cu") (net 16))
 (segment (start 138.12 81.395) (end 139.3703 81.395) (width 0.4) (layer "B.Cu") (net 16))
 (segment (start 139.3703 80.8769) (end 139.3703 81.395) (width 0.4) (layer "B.Cu") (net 16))
 (segment (start 130.5 81.395) (end 131.7503 81.395) (width 0.4) (layer "F.Cu") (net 13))
 (segment (start 143.7905 78.2154) (end 140.3338 78.2154) (width 0.4) (layer "F.Cu") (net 13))
 (segment (start 145.6056 76.4003) (end 143.7905 78.2154) (width 0.4) (layer "F.Cu") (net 13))
 (segment (start 146.25 73.5) (end 146.25 76.4003) (width 0.4) (layer "F.Cu") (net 13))
 (segment (start 132.4907 80.1365) (end 131.7503 80.8769) (width 0.4) (layer "F.Cu") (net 13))
 (segment (start 139.013 79.5362) (end 136.9211 79.5362) (width 0.4) (layer "F.Cu") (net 13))
 (segment (start 136.9211 79.5362) (end 136.3208 80.1365) (width 0.4) (layer "F.Cu") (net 13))
 (segment (start 131.7503 80.8769) (end 131.7503 81.395) (width 0.4) (layer "F.Cu") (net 13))
 (segment (start 146.25 76.4003) (end 145.6056 76.4003) (width 0.4) (layer "F.Cu") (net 13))
 (segment (start 140.3338 78.2154) (end 139.013 79.5362) (width 0.4) (layer "F.Cu") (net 13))
 (segment (start 136.3208 80.1365) (end 132.4907 80.1365) (width 0.4) (layer "F.Cu") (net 13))
 (segment (start 147.75 76.4003) (end 146.8312 77.3191) (width 0.4) (layer "F.Cu") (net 14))
 (segment (start 147.75 73.5) (end 147.75 76.4003) (width 0.4) (layer "F.Cu") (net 14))
 (segment (start 146.8312 77.3191) (end 145.8185 77.3191) (width 0.4) (layer "F.Cu") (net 14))
 (via (at 145.8185 77.3191) (size 0.8) (drill 0.4) (layers "F.Cu" "B.Cu") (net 14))
 (segment (start 143.9256 79.212) (end 135.9552 79.212) (width 0.4) (layer "B.Cu") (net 14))
 (segment (start 145.8185 77.3191) (end 143.9256 79.212) (width 0.4) (layer "B.Cu") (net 14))
 (segment (start 135.9552 79.212) (end 134.2903 80.8769) (width 0.4) (layer "B.Cu") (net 14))
 (segment (start 133.04 81.395) (end 134.2903 81.395) (width 0.4) (layer "B.Cu") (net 14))
 (segment (start 134.2903 80.8769) (end 134.2903 81.395) (width 0.4) (layer "B.Cu") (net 14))
 (segment (start 143.25 73.5) (end 143.25 76.4003) (width 0.4) (layer "F.Cu") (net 11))
 (segment (start 142.3632 77.2871) (end 141.436 77.2871) (width 0.4) (layer "F.Cu") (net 11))
 (segment (start 143.25 76.4003) (end 142.3632 77.2871) (width 0.4) (layer "F.Cu") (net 11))
 (via (at 141.436 77.2871) (size 0.8) (drill 0.4) (layers "F.Cu" "B.Cu") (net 11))
 (segment (start 126.6703 80.8769) (end 126.6703 81.395) (width 0.4) (layer "B.Cu") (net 11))
 (segment (start 130.2601 77.2871) (end 126.6703 80.8769) (width 0.4) (layer "B.Cu") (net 11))
 (segment (start 125.42 81.395) (end 126.6703 81.395) (width 0.4) (layer "B.Cu") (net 11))
 (segment (start 141.436 77.2871) (end 130.2601 77.2871) (width 0.4) (layer "B.Cu") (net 11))
 (segment (start 144.75 73.5) (end 144.75 76.4003) (width 0.4) (layer "F.Cu") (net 12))
 (segment (start 144.75 76.4003) (end 144.3418 76.4003) (width 0.4) (layer "F.Cu") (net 12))
 (segment (start 144.3418 76.4003) (end 144.0878 76.6543) (width 0.4) (layer "F.Cu") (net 12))
 (via (at 144.0878 76.6543) (size 0.8) (drill 0.4) (layers "F.Cu" "B.Cu") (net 12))
 (segment (start 131.9544 78.1039) (end 129.2103 80.848) (width 0.4) (layer "B.Cu") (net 12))
 (segment (start 142.6382 78.1039) (end 131.9544 78.1039) (width 0.4) (layer "B.Cu") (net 12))
 (segment (start 127.96 81.395) (end 129.2103 81.395) (width 0.4) (layer "B.Cu") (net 12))
 (segment (start 129.2103 80.848) (end 129.2103 81.395) (width 0.4) (layer "B.Cu") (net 12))
 (segment (start 144.0878 76.6543) (end 142.6382 78.1039) (width 0.4) (layer "B.Cu") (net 12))
 (segment (start 138.3147 78.3356) (end 136.4239 78.3356) (width 0.4) (layer "F.Cu") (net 9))
 (segment (start 140.25 73.5) (end 140.25 76.4003) (width 0.4) (layer "F.Cu") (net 9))
 (segment (start 120.34 81.395) (end 121.5903 81.395) (width 0.4) (layer "F.Cu") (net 9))
 (segment (start 140.25 76.4003) (end 138.3147 78.3356) (width 0.4) (layer "F.Cu") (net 9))
 (segment (start 123.5314 78.9358) (end 121.5903 80.8769) (width 0.4) (layer "F.Cu") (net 9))
 (segment (start 136.4239 78.3356) (end 135.8237 78.9358) (width 0.4) (layer "F.Cu") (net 9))
 (segment (start 121.5903 80.8769) (end 121.5903 81.395) (width 0.4) (layer "F.Cu") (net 9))
 (segment (start 135.8237 78.9358) (end 123.5314 78.9358) (width 0.4) (layer "F.Cu") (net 9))
 (segment (start 141.1693 76.4003) (end 138.6337 78.9359) (width 0.4) (layer "F.Cu") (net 10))
 (segment (start 124.1303 80.8769) (end 124.1303 81.395) (width 0.4) (layer "F.Cu") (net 10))
 (segment (start 136.0723 79.5361) (end 125.4711 79.5361) (width 0.4) (layer "F.Cu") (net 10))
 (segment (start 141.75 76.4003) (end 141.1693 76.4003) (width 0.4) (layer "F.Cu") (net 10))
 (segment (start 136.6725 78.9359) (end 136.0723 79.5361) (width 0.4) (layer "F.Cu") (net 10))
 (segment (start 141.75 73.5) (end 141.75 76.4003) (width 0.4) (layer "F.Cu") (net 10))
 (segment (start 138.6337 78.9359) (end 136.6725 78.9359) (width 0.4) (layer "F.Cu") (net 10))
 (segment (start 125.4711 79.5361) (end 124.1303 80.8769) (width 0.4) (layer "F.Cu") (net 10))
 (segment (start 122.88 81.395) (end 124.1303 81.395) (width 0.4) (layer "F.Cu") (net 10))
 (segment (start 137.25 73.5) (end 137.25 76.4003) (width 0.4) (layer "F.Cu") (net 7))
 (segment (start 137.25 76.4003) (end 136.6614 76.4003) (width 0.4) (layer "F.Cu") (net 7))
 (segment (start 135.4606 77.6011) (end 119.7861 77.6011) (width 0.4) (layer "F.Cu") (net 7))
 (segment (start 136.6614 76.4003) (end 135.4606 77.6011) (width 0.4) (layer "F.Cu") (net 7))
 (segment (start 119.7861 77.6011) (end 116.5103 80.8769) (width 0.4) (layer "F.Cu") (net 7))
 (segment (start 115.26 81.395) (end 116.5103 81.395) (width 0.4) (layer "F.Cu") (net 7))
 (segment (start 116.5103 80.8769) (end 116.5103 81.395) (width 0.4) (layer "F.Cu") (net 7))
 (segment (start 117.8 81.395) (end 119.0503 81.395) (width 0.4) (layer "F.Cu") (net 8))
 (segment (start 135.7091 78.2015) (end 121.7257 78.2015) (width 0.4) (layer "F.Cu") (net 8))
 (segment (start 121.7257 78.2015) (end 119.0503 80.8769) (width 0.4) (layer "F.Cu") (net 8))
 (segment (start 137.415 77.7353) (end 136.1753 77.7353) (width 0.4) (layer "F.Cu") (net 8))
 (segment (start 138.75 76.4003) (end 137.415 77.7353) (width 0.4) (layer "F.Cu") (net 8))
 (segment (start 136.1753 77.7353) (end 135.7091 78.2015) (width 0.4) (layer "F.Cu") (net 8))
 (segment (start 119.0503 80.8769) (end 119.0503 81.395) (width 0.4) (layer "F.Cu") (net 8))
 (segment (start 138.75 73.5) (end 138.75 76.4003) (width 0.4) (layer "F.Cu") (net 8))
 (segment (start 134.25 76.4003) (end 115.9069 76.4003) (width 0.4) (layer "F.Cu") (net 5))
 (segment (start 115.9069 76.4003) (end 111.4303 80.8769) (width 0.4) (layer "F.Cu") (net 5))
 (segment (start 110.18 81.395) (end 111.4303 81.395) (width 0.4) (layer "F.Cu") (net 5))
 (segment (start 134.25 73.5) (end 134.25 76.4003) (width 0.4) (layer "F.Cu") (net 5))
 (segment (start 111.4303 80.8769) (end 111.4303 81.395) (width 0.4) (layer "F.Cu") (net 5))
 (segment (start 135.75 76.4003) (end 135.1496 77.0007) (width 0.4) (layer "F.Cu") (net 6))
 (segment (start 135.75 73.5) (end 135.75 76.4003) (width 0.4) (layer "F.Cu") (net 6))
 (segment (start 112.72 81.395) (end 113.9703 81.395) (width 0.4) (layer "F.Cu") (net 6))
 (segment (start 135.1496 77.0007) (end 117.8465 77.0007) (width 0.4) (layer "F.Cu") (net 6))
 (segment (start 117.8465 77.0007) (end 113.9703 80.8769) (width 0.4) (layer "F.Cu") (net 6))
 (segment (start 113.9703 80.8769) (end 113.9703 81.395) (width 0.4) (layer "F.Cu") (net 6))
 (segment (start 157.1503 80.5) (end 157.1503 81.395) (width 0.4) (layer "F.Cu") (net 23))
 (segment (start 155.9 81.395) (end 157.1503 81.395) (width 0.4) (layer "F.Cu") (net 23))
 (segment (start 161.25 76.4003) (end 157.1503 80.5) (width 0.4) (layer "F.Cu") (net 23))
 (segment (start 161.25 73.5) (end 161.25 76.4003) (width 0.4) (layer "F.Cu") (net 23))
 (segment (start 128.25 73.5) (end 128.25 70.5997) (width 0.4) (layer "F.Cu") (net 30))
 (segment (start 129.1775 69.6722) (end 129.5079 69.6722) (width 0.4) (layer "F.Cu") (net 30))
 (segment (start 128.25 70.5997) (end 129.1775 69.6722) (width 0.4) (layer "F.Cu") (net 30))
 (via (at 129.5079 69.6722) (size 0.8) (drill 0.4) (layers "F.Cu" "B.Cu") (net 30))
 (segment (start 161.225 69.6722) (end 172.4297 80.8769) (width 0.4) (layer "B.Cu") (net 30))
 (segment (start 173.68 81.395) (end 172.4297 81.395) (width 0.4) (layer "B.Cu") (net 30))
 (segment (start 172.4297 80.8769) (end 172.4297 81.395) (width 0.4) (layer "B.Cu") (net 30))
 (segment (start 129.5079 69.6722) (end 161.225 69.6722) (width 0.4) (layer "B.Cu") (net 30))
 (segment (start 107.2262 50.6995) (end 105.1 52.8257) (width 0.7) (layer "B.Cu") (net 3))
 (segment (start 114.7 51.1997) (end 114.1998 50.6995) (width 0.7) (layer "B.Cu") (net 3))
 (segment (start 114.7 53) (end 114.7 51.1997) (width 0.7) (layer "B.Cu") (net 3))
 (segment (start 114.1998 50.6995) (end 107.2262 50.6995) (width 0.7) (layer "B.Cu") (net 3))
 (segment (start 105.1 52.8257) (end 105.1 81.395) (width 0.7) (layer "B.Cu") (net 3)))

